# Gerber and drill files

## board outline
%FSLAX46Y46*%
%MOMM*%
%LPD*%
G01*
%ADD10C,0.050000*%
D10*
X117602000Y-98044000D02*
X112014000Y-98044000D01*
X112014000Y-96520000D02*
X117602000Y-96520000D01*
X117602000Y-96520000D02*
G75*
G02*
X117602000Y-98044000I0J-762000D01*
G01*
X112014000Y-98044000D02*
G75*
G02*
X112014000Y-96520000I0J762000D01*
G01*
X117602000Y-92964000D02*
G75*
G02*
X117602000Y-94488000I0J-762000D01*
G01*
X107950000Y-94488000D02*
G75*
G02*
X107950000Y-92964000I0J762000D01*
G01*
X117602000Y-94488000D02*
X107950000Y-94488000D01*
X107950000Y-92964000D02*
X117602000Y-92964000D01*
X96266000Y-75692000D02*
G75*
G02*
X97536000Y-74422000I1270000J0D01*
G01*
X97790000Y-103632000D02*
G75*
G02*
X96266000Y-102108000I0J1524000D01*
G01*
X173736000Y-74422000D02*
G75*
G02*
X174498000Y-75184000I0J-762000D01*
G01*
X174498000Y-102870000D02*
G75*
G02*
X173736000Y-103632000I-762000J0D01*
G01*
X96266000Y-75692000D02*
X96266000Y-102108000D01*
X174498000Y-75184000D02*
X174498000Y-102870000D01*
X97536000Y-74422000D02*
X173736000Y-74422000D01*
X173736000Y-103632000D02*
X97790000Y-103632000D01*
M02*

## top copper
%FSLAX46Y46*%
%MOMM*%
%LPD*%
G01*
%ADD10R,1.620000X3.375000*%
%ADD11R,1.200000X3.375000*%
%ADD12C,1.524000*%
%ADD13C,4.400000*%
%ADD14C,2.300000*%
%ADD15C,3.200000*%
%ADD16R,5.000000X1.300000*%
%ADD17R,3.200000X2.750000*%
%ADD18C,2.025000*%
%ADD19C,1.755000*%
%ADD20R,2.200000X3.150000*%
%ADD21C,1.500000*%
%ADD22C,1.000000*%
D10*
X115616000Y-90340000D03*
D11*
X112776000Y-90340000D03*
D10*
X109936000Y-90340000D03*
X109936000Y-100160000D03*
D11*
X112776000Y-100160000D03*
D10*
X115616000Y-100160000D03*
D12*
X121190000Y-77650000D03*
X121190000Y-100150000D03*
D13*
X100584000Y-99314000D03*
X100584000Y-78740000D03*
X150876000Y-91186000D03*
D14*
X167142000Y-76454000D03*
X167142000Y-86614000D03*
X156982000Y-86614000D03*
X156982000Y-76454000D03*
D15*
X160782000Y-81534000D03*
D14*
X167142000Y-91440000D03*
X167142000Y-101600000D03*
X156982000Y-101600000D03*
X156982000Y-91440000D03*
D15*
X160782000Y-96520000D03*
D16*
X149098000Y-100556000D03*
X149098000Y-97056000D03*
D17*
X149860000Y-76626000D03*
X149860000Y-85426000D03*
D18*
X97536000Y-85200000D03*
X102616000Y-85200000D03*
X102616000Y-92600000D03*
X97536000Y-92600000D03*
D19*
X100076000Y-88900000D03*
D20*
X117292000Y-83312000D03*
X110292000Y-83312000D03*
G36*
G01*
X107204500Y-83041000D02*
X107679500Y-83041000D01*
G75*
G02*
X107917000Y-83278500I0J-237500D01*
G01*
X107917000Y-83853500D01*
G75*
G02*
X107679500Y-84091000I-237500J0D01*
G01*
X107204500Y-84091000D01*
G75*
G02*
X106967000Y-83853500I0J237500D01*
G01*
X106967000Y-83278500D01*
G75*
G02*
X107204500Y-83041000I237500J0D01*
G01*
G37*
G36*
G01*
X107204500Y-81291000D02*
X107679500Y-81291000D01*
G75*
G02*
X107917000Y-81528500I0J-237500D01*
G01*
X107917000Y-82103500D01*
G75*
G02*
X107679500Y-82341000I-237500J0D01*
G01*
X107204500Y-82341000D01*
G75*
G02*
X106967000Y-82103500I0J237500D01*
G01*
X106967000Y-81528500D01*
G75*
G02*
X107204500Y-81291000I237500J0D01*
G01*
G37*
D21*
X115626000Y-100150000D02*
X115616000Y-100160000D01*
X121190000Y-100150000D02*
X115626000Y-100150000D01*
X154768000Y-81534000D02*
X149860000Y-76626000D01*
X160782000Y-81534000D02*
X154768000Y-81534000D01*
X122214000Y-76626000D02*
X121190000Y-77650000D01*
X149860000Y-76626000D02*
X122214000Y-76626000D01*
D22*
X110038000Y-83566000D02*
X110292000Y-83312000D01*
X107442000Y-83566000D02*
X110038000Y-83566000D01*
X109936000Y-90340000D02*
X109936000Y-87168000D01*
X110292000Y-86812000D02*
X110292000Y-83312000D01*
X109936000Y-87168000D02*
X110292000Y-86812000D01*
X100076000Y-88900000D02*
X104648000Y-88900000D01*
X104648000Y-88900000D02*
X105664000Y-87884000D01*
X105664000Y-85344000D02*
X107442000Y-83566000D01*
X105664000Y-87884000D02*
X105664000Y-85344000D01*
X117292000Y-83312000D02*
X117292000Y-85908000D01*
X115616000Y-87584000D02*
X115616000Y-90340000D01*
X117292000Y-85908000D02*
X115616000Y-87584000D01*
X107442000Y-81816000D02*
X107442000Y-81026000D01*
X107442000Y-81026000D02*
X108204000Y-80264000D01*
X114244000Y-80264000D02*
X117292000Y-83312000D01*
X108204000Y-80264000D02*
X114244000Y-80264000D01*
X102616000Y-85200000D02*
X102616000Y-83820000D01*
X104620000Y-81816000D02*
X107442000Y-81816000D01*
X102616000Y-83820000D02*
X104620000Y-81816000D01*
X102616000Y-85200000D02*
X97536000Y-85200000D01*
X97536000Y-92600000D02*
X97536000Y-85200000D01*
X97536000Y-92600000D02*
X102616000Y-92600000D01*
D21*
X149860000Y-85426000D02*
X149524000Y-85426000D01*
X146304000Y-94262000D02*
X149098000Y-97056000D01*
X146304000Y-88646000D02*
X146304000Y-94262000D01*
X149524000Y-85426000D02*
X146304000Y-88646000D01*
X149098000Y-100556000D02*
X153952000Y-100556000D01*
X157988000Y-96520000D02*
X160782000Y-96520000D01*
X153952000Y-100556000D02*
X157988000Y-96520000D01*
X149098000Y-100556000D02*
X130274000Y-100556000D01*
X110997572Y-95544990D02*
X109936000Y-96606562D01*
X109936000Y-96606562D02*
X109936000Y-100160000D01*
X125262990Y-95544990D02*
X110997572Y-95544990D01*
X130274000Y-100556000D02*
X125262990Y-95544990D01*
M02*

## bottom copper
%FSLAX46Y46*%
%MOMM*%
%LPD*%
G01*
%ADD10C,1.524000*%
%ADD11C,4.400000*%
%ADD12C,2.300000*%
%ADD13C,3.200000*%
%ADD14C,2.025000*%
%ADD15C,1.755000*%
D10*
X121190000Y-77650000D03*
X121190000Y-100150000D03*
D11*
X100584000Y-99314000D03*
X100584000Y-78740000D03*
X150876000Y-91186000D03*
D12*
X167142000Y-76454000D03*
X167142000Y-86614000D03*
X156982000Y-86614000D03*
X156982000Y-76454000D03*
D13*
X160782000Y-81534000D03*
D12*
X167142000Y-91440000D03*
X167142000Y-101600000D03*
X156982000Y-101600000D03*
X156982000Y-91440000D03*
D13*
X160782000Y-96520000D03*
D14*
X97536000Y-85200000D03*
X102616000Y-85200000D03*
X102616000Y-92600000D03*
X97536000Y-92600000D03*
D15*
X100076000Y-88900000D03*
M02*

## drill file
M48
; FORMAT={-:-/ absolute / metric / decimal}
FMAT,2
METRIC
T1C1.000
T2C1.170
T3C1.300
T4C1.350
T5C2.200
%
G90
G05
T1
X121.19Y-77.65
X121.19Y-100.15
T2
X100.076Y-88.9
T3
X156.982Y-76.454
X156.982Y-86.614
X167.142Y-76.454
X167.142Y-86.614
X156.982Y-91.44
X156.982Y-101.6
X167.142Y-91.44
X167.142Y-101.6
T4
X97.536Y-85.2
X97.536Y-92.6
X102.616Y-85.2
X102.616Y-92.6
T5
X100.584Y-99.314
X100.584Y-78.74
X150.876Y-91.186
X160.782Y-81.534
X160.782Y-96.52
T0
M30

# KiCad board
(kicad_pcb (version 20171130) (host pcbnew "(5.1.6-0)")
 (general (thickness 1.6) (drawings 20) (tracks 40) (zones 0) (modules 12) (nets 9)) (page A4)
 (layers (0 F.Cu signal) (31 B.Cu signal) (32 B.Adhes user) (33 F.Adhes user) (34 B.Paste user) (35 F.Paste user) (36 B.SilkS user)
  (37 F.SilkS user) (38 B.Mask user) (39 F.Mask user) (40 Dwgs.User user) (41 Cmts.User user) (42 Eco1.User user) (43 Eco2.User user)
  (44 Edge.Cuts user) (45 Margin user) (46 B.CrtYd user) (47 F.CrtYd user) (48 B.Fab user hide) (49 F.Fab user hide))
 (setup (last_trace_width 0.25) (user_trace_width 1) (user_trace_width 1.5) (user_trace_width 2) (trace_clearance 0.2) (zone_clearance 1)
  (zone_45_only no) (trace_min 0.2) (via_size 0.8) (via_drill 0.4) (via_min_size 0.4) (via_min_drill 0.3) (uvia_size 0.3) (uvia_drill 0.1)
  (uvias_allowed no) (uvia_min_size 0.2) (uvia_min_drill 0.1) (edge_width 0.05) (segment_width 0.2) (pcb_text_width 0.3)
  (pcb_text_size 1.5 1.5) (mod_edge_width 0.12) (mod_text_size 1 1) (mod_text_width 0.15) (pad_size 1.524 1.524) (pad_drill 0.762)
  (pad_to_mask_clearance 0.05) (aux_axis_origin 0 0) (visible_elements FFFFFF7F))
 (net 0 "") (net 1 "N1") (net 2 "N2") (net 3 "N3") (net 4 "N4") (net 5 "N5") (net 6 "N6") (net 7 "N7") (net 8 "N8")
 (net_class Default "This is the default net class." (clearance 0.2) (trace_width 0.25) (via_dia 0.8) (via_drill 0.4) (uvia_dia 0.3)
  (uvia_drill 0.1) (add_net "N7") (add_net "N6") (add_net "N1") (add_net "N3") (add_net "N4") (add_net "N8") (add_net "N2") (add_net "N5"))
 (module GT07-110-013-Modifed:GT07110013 (layer F.Cu) (at 112.776 95.25)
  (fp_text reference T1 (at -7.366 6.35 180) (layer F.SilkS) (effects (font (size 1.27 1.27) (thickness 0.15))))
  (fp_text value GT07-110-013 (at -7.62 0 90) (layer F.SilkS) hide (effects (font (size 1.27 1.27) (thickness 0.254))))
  (pad 1 smd rect (at 2.84 -4.91) (size 1.62 3.375) (layers F.Cu F.Paste F.Mask) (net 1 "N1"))
  (pad 2 smd rect (at 0 -4.91) (size 1.2 3.375) (layers F.Cu F.Paste F.Mask) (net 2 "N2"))
  (pad 3 smd rect (at -2.84 -4.91) (size 1.62 3.375) (layers F.Cu F.Paste F.Mask) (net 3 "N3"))
  (pad 4 smd rect (at -2.84 4.91) (size 1.62 3.375) (layers F.Cu F.Paste F.Mask) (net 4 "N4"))
  (pad 5 smd rect (at 0 4.91) (size 1.2 3.375) (layers F.Cu F.Paste F.Mask) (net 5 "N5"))
  (pad 6 smd rect (at 2.84 4.91) (size 1.62 3.375) (layers F.Cu F.Paste F.Mask) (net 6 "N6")))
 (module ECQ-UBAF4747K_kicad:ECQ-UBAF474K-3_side (layer F.Cu) (at 123.19 88.9 180)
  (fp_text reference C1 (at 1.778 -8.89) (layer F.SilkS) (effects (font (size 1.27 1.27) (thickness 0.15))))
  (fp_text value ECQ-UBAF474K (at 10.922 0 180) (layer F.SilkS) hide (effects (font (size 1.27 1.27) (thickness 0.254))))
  (pad 1 thru_hole circle (at 2 11.25 180) (size 1.524 1.524) (drill 1) (layers *.Cu *.Mask) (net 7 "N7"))
  (pad 2 thru_hole circle (at 2 -11.25 180) (size 1.524 1.524) (drill 1) (layers *.Cu *.Mask) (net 6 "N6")))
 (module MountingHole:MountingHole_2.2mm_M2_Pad (layer F.Cu) (at 100.584 99.314)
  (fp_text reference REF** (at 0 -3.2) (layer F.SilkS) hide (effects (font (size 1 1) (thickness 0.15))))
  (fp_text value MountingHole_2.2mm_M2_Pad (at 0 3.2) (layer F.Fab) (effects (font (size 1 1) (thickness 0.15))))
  (pad 1 thru_hole circle (at 0 0) (size 4.4 4.4) (drill 2.2) (layers *.Cu *.Mask)))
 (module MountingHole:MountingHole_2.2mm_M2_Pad (layer F.Cu) (at 100.584 78.74)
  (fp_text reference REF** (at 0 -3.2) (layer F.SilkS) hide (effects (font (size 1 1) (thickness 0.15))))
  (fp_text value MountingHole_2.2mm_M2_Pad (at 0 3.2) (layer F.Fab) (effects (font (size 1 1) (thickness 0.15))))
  (pad 1 thru_hole circle (at 0 0) (size 4.4 4.4) (drill 2.2) (layers *.Cu *.Mask)))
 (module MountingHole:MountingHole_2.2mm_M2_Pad (layer F.Cu) (at 150.876 91.186)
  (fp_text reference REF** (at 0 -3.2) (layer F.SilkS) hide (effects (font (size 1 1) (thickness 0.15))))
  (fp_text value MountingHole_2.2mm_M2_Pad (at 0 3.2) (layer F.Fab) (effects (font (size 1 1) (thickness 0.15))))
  (pad 1 thru_hole circle (at 0 0) (size 4.4 4.4) (drill 2.2) (layers *.Cu *.Mask)))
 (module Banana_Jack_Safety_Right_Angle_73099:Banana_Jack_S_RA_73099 (layer F.Cu) (at 160.782 81.534)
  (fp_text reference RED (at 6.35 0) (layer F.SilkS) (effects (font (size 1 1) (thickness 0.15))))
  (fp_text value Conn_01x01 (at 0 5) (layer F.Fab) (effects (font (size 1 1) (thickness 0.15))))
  (pad 2 thru_hole circle (at 6.36 -5.08) (size 2.3 2.3) (drill 1.3) (layers *.Cu *.Mask))
  (pad 2 thru_hole circle (at 6.36 5.08) (size 2.3 2.3) (drill 1.3) (layers *.Cu *.Mask))
  (pad 2 thru_hole circle (at -3.8 5.08) (size 2.3 2.3) (drill 1.3) (layers *.Cu *.Mask))
  (pad 2 thru_hole circle (at -3.8 -5.08) (size 2.3 2.3) (drill 1.3) (layers *.Cu *.Mask))
  (pad 1 thru_hole circle (at 0 0) (size 3.2 3.2) (drill 2.2) (layers *.Cu *.Mask) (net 7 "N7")))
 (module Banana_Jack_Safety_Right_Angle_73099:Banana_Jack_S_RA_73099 (layer F.Cu) (at 160.782 96.52)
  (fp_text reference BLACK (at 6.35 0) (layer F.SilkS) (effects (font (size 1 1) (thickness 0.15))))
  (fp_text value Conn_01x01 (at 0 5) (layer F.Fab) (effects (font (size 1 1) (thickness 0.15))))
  (pad 2 thru_hole circle (at 6.36 -5.08) (size 2.3 2.3) (drill 1.3) (layers *.Cu *.Mask))
  (pad 2 thru_hole circle (at 6.36 5.08) (size 2.3 2.3) (drill 1.3) (layers *.Cu *.Mask))
  (pad 2 thru_hole circle (at -3.8 5.08) (size 2.3 2.3) (drill 1.3) (layers *.Cu *.Mask))
  (pad 2 thru_hole circle (at -3.8 -5.08) (size 2.3 2.3) (drill 1.3) (layers *.Cu *.Mask))
  (pad 1 thru_hole circle (at 0 0) (size 3.2 3.2) (drill 2.2) (layers *.Cu *.Mask) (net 4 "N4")))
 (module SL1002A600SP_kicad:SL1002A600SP (layer F.Cu) (at 149.098 98.806 270)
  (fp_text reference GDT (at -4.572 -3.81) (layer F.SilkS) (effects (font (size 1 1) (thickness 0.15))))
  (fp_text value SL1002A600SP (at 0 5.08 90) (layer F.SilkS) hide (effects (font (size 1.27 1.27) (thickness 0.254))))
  (pad 2 smd rect (at 1.75 0 270) (size 1.3 5) (layers F.Cu F.Paste F.Mask) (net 4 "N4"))
  (pad 1 smd rect (at -1.75 0 270) (size 1.3 5) (layers F.Cu F.Paste F.Mask) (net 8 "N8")))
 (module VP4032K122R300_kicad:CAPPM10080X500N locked (layer F.Cu) (at 149.86 81.026 90)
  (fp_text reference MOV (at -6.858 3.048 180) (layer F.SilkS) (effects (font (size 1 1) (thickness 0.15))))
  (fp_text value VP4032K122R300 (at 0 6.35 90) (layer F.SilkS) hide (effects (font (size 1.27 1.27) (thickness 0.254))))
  (pad 2 smd rect (at 4.4 0 90) (size 2.75 3.2) (layers F.Cu F.Paste F.Mask) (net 7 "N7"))
  (pad 1 smd rect (at -4.4 0 90) (size 2.75 3.2) (layers F.Cu F.Paste F.Mask) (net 8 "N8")))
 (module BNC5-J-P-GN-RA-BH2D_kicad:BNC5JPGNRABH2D (layer F.Cu) (at 100.076 88.9 90)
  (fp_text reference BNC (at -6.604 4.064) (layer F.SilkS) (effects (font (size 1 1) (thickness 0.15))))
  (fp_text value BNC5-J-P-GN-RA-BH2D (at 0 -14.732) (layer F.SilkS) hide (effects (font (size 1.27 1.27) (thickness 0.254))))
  (pad 5 thru_hole circle (at 3.7 -2.54 90) (size 2.025 2.025) (drill 1.35) (layers *.Cu *.Mask) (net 1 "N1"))
  (pad 4 thru_hole circle (at 3.7 2.54 90) (size 2.025 2.025) (drill 1.35) (layers *.Cu *.Mask) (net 1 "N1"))
  (pad 3 thru_hole circle (at -3.7 2.54 90) (size 2.025 2.025) (drill 1.35) (layers *.Cu *.Mask) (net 1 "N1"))
  (pad 2 thru_hole circle (at -3.7 -2.54 90) (size 2.025 2.025) (drill 1.35) (layers *.Cu *.Mask) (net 1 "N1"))
  (pad 1 thru_hole circle (at 0 0 90) (size 1.755 1.755) (drill 1.17) (layers *.Cu *.Mask) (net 3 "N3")))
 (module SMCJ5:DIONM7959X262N (layer F.Cu) (at 113.792 83.312)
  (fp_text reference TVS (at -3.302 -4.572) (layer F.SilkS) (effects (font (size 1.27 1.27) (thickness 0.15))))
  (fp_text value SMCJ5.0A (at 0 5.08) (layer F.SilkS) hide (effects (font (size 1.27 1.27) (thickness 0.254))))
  (pad 2 smd rect (at 3.5 0) (size 2.2 3.15) (layers F.Cu F.Paste F.Mask) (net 1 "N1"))
  (pad 1 smd rect (at -3.5 0) (size 2.2 3.15) (layers F.Cu F.Paste F.Mask) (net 3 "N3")))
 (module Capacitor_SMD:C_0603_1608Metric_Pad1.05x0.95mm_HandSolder (layer F.Cu) (at 107.442 82.691 270)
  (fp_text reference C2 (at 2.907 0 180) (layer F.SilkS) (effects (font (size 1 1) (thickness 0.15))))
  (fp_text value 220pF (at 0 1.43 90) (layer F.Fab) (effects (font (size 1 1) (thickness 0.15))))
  (pad 2 smd roundrect (at 0.875 0 270) (size 1.05 0.95) (layers F.Cu F.Paste F.Mask) (roundrect_rratio 0.25) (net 3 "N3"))
  (pad 1 smd roundrect (at -0.875 0 270) (size 1.05 0.95) (layers F.Cu F.Paste F.Mask) (roundrect_rratio 0.25) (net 1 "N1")))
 (gr_line (start 117.602 98.044) (end 112.014 98.044) (layer Edge.Cuts) (width 0.05))
 (gr_line (start 112.014 96.52) (end 117.602 96.52) (layer Edge.Cuts) (width 0.05))
 (gr_arc (start 117.602 97.282) (end 117.602 98.044) (angle -180) (layer Edge.Cuts) (width 0.05))
 (gr_arc (start 112.014 97.282) (end 112.014 96.52) (angle -180) (layer Edge.Cuts) (width 0.05))
 (gr_arc (start 117.602 93.726) (end 117.602 94.488) (angle -180) (layer Edge.Cuts) (width 0.05))
 (gr_arc (start 107.95 93.726) (end 107.95 92.964) (angle -180) (layer Edge.Cuts) (width 0.05))
 (gr_line (start 117.602 94.488) (end 107.95 94.488) (layer Edge.Cuts) (width 0.05))
 (gr_line (start 107.95 92.964) (end 117.602 92.964) (layer Edge.Cuts) (width 0.05))
 (gr_arc (start 97.536 75.692) (end 97.536 74.422) (angle -90) (layer Edge.Cuts) (width 0.05))
 (gr_arc (start 97.79 102.108) (end 96.266 102.108) (angle -90) (layer Edge.Cuts) (width 0.05))
 (gr_arc (start 173.736 75.184) (end 174.498 75.184) (angle -90) (layer Edge.Cuts) (width 0.05))
 (gr_arc (start 173.736 102.87) (end 173.736 103.632) (angle -90) (layer Edge.Cuts) (width 0.05))
 (gr_line (start 96.266 75.692) (end 96.266 102.108) (layer Edge.Cuts) (width 0.05))
 (gr_line (start 174.498 75.184) (end 174.498 102.87) (layer Edge.Cuts) (width 0.05))
 (gr_line (start 97.536 74.422) (end 173.736 74.422) (layer Edge.Cuts) (width 0.05))
 (gr_line (start 173.736 103.632) (end 97.79 103.632) (layer Edge.Cuts) (width 0.05))
 (segment (start 115.626 100.15) (end 115.616 100.16) (width 1.5) (layer F.Cu) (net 6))
 (segment (start 121.19 100.15) (end 115.626 100.15) (width 1.5) (layer F.Cu) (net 6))
 (segment (start 154.768 81.534) (end 149.86 76.626) (width 1.5) (layer F.Cu) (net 7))
 (segment (start 160.782 81.534) (end 154.768 81.534) (width 1.5) (layer F.Cu) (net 7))
 (segment (start 122.214 76.626) (end 121.19 77.65) (width 1.5) (layer F.Cu) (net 7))
 (segment (start 149.86 76.626) (end 122.214 76.626) (width 1.5) (layer F.Cu) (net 7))
 (segment (start 110.038 83.566) (end 110.292 83.312) (width 1) (layer F.Cu) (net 3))
 (segment (start 107.442 83.566) (end 110.038 83.566) (width 1) (layer F.Cu) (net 3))
 (segment (start 109.936 90.34) (end 109.936 87.168) (width 1) (layer F.Cu) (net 3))
 (segment (start 110.292 86.812) (end 110.292 83.312) (width 1) (layer F.Cu) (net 3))
 (segment (start 109.936 87.168) (end 110.292 86.812) (width 1) (layer F.Cu) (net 3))
 (segment (start 100.076 88.9) (end 104.648 88.9) (width 1) (layer F.Cu) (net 3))
 (segment (start 104.648 88.9) (end 105.664 87.884) (width 1) (layer F.Cu) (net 3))
 (segment (start 105.664 85.344) (end 107.442 83.566) (width 1) (layer F.Cu) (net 3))
 (segment (start 105.664 87.884) (end 105.664 85.344) (width 1) (layer F.Cu) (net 3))
 (segment (start 117.292 83.312) (end 117.292 85.908) (width 1) (layer F.Cu) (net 1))
 (segment (start 115.616 87.584) (end 115.616 90.34) (width 1) (layer F.Cu) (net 1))
 (segment (start 117.292 85.908) (end 115.616 87.584) (width 1) (layer F.Cu) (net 1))
 (segment (start 107.442 81.816) (end 107.442 81.026) (width 1) (layer F.Cu) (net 1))
 (segment (start 107.442 81.026) (end 108.204 80.264) (width 1) (layer F.Cu) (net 1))
 (segment (start 114.244 80.264) (end 117.292 83.312) (width 1) (layer F.Cu) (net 1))
 (segment (start 108.204 80.264) (end 114.244 80.264) (width 1) (layer F.Cu) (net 1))
 (segment (start 102.616 85.2) (end 102.616 83.82) (width 1) (layer F.Cu) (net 1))
 (segment (start 104.62 81.816) (end 107.442 81.816) (width 1) (layer F.Cu) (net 1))
 (segment (start 102.616 83.82) (end 104.62 81.816) (width 1) (layer F.Cu) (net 1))
 (segment (start 102.616 85.2) (end 97.536 85.2) (width 1) (layer F.Cu) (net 1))
 (segment (start 97.536 92.6) (end 97.536 85.2) (width 1) (layer F.Cu) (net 1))
 (segment (start 97.536 92.6) (end 102.616 92.6) (width 1) (layer F.Cu) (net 1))
 (segment (start 149.86 85.426) (end 149.524 85.426) (width 1.5) (layer F.Cu) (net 8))
 (segment (start 146.304 94.262) (end 149.098 97.056) (width 1.5) (layer F.Cu) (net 8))
 (segment (start 146.304 88.646) (end 146.304 94.262) (width 1.5) (layer F.Cu) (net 8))
 (segment (start 149.524 85.426) (end 146.304 88.646) (width 1.5) (layer F.Cu) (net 8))
 (segment (start 149.098 100.556) (end 153.952 100.556) (width 1.5) (layer F.Cu) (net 4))
 (segment (start 157.988 96.52) (end 160.782 96.52) (width 1.5) (layer F.Cu) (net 4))
 (segment (start 153.952 100.556) (end 157.988 96.52) (width 1.5) (layer F.Cu) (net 4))
 (segment (start 149.098 100.556) (end 130.274 100.556) (width 1.5) (layer F.Cu) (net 4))
 (segment (start 110.997572 95.54499) (end 109.936 96.606562) (width 1.5) (layer F.Cu) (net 4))
 (segment (start 109.936 96.606562) (end 109.936 100.16) (width 1.5) (layer F.Cu) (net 4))
 (segment (start 125.26299 95.54499) (end 110.997572 95.54499) (width 1.5) (layer F.Cu) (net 4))
 (segment (start 130.274 100.556) (end 125.26299 95.54499) (width 1.5) (layer F.Cu) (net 4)))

